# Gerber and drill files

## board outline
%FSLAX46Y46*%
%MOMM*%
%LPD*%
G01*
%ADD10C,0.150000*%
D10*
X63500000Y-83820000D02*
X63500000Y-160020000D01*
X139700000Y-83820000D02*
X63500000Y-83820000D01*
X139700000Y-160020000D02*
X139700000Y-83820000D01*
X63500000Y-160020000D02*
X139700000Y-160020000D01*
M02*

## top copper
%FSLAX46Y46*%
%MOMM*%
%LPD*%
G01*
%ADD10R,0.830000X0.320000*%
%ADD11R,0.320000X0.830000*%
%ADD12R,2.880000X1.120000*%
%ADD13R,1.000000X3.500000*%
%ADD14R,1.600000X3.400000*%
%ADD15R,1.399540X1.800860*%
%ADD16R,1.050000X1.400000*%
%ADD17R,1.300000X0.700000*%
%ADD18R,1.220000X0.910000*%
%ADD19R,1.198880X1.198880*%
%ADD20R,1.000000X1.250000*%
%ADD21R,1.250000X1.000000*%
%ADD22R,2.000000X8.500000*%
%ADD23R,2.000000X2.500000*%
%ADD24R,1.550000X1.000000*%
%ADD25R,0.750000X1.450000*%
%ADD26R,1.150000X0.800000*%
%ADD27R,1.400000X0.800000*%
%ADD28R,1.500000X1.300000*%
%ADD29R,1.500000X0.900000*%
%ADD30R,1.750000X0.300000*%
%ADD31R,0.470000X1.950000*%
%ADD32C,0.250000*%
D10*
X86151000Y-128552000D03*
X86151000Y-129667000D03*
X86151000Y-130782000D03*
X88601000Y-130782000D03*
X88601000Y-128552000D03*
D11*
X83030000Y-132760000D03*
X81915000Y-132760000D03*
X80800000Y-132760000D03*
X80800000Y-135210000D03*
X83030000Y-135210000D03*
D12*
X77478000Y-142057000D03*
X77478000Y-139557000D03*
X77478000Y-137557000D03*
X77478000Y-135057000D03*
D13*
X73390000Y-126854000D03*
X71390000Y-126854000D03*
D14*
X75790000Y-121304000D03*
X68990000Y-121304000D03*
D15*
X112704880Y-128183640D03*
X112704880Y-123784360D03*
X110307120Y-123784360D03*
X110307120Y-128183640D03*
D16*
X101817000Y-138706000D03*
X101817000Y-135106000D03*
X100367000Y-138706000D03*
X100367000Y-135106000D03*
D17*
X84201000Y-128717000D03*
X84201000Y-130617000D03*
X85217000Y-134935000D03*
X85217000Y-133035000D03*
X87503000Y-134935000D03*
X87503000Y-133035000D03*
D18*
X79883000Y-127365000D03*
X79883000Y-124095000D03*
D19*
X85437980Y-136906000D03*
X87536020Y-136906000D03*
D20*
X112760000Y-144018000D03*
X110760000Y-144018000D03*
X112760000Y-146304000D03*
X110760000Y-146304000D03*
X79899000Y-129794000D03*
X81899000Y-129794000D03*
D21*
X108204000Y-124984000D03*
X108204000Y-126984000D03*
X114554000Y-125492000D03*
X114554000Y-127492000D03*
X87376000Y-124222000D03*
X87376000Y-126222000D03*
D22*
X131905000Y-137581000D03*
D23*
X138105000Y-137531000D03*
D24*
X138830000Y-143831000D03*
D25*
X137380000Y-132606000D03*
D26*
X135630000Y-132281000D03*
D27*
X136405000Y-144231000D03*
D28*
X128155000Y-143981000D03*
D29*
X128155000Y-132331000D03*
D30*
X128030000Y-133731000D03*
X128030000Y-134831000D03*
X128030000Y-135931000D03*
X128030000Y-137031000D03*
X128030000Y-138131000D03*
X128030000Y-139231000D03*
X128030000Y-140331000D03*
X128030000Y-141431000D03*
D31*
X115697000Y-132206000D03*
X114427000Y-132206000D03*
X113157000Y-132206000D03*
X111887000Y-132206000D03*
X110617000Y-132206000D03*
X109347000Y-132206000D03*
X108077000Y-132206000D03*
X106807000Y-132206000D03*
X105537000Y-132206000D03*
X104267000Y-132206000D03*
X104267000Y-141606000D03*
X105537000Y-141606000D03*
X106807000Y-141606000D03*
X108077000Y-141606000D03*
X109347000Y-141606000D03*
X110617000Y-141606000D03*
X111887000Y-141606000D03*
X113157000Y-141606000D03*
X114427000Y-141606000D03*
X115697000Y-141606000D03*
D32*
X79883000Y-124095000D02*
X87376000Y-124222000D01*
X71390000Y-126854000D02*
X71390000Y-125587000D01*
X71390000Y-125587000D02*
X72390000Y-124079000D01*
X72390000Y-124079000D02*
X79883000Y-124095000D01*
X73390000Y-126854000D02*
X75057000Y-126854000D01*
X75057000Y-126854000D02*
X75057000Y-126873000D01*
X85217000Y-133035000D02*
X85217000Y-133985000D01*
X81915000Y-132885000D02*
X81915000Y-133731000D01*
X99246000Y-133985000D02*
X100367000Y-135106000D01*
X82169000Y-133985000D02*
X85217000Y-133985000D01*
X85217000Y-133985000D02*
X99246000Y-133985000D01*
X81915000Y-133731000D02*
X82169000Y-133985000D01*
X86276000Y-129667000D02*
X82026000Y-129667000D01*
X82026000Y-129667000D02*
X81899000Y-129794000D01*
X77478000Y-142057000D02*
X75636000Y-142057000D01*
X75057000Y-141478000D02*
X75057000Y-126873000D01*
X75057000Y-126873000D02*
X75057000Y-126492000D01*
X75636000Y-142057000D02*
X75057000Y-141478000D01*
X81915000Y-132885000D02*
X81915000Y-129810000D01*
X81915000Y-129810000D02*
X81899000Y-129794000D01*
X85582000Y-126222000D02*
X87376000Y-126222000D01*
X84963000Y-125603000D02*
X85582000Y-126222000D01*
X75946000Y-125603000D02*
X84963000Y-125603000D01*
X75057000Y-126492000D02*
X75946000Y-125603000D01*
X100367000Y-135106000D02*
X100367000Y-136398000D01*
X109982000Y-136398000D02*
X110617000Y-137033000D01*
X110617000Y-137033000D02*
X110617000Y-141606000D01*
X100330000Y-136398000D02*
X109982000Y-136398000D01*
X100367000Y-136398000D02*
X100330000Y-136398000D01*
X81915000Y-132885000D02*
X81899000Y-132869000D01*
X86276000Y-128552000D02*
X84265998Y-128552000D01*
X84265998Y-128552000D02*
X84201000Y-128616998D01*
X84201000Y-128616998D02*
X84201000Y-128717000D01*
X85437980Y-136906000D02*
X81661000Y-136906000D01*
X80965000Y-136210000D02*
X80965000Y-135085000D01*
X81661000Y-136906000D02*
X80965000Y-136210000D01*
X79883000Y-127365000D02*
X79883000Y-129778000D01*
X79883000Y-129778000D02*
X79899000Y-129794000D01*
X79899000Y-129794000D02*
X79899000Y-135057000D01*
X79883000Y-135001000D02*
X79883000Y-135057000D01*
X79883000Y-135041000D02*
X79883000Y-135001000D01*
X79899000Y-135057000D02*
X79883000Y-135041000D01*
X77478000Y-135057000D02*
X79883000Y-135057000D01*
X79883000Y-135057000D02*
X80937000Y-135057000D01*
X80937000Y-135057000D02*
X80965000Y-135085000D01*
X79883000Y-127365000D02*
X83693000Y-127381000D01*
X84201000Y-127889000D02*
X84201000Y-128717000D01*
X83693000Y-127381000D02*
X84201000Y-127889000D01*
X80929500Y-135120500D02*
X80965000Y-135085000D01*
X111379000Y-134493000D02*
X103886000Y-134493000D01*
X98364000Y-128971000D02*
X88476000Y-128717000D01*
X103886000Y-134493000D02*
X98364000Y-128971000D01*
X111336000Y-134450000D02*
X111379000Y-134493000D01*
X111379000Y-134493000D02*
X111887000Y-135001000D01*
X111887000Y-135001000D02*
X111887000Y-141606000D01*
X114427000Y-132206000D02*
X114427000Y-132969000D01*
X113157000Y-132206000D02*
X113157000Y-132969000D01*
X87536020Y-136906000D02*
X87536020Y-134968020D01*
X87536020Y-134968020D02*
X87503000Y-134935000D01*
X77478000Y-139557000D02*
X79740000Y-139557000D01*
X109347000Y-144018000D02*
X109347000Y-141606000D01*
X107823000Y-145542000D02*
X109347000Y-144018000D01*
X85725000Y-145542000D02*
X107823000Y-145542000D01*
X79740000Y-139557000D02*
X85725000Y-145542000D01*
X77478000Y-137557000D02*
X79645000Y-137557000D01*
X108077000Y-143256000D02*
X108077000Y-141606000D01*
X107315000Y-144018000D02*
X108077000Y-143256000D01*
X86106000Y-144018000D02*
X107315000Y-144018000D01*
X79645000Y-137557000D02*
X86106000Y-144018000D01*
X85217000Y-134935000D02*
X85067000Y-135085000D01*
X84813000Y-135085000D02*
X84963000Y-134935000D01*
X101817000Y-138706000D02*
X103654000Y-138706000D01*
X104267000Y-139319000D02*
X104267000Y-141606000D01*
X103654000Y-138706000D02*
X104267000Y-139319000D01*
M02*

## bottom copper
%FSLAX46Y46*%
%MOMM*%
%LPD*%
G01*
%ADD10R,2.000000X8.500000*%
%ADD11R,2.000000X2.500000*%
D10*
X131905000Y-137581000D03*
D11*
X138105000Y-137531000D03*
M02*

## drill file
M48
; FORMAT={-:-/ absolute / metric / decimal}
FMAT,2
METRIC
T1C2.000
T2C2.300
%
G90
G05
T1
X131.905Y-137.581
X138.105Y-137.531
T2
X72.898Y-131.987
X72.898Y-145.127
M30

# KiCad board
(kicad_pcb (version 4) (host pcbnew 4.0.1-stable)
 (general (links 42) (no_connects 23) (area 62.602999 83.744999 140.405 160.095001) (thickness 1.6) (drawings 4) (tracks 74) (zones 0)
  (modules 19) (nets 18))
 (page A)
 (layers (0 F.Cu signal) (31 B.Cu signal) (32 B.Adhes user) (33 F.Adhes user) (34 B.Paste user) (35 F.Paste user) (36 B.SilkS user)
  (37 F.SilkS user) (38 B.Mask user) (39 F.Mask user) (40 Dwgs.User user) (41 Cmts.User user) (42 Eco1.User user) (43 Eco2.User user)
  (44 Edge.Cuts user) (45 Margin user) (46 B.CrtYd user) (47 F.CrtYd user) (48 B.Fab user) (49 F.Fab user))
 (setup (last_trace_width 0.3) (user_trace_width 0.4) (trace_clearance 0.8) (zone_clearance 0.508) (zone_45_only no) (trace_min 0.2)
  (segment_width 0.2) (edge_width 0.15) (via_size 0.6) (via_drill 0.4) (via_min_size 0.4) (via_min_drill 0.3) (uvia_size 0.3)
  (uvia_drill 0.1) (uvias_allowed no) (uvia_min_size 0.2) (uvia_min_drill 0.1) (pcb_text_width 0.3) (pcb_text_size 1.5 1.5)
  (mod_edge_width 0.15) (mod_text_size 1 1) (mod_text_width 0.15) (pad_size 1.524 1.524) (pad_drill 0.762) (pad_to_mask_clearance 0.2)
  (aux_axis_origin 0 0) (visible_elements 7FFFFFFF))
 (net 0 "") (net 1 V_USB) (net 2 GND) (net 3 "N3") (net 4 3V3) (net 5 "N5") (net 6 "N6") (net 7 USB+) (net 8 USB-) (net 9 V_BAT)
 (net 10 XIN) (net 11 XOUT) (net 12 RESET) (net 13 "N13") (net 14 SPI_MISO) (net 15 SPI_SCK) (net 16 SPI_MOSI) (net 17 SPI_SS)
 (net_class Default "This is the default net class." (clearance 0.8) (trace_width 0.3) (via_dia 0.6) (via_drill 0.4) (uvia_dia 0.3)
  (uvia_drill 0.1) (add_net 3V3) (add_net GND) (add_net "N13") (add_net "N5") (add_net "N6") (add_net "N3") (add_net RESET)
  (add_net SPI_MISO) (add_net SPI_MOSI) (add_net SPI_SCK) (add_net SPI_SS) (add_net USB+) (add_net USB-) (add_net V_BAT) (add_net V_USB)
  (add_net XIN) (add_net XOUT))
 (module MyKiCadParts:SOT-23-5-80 (layer F.Cu) (at 87.376 129.667)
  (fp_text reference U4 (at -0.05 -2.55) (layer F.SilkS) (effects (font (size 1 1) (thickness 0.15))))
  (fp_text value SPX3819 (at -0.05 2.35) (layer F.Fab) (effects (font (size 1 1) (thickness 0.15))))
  (pad 1 smd rect (at -1.225 -1.115) (size 0.83 0.32) (layers F.Cu F.Paste F.Mask) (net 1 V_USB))
  (pad 2 smd rect (at -1.225 0) (size 0.83 0.32) (layers F.Cu F.Paste F.Mask) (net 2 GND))
  (pad 3 smd rect (at -1.225 1.115) (size 0.83 0.32) (layers F.Cu F.Paste F.Mask) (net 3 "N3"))
  (pad 4 smd rect (at 1.225 1.115) (size 0.83 0.32) (layers F.Cu F.Paste F.Mask))
  (pad 5 smd rect (at 1.225 -1.115) (size 0.83 0.32) (layers F.Cu F.Paste F.Mask) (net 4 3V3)))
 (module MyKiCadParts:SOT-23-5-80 (layer F.Cu) (at 81.915 133.985 270)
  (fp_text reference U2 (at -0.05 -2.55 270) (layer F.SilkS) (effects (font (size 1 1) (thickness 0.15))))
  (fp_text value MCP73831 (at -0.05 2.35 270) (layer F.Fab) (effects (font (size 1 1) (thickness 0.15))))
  (pad 1 smd rect (at -1.225 -1.115 270) (size 0.83 0.32) (layers F.Cu F.Paste F.Mask) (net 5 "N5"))
  (pad 2 smd rect (at -1.225 0 270) (size 0.83 0.32) (layers F.Cu F.Paste F.Mask) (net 2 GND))
  (pad 3 smd rect (at -1.225 1.115 270) (size 0.83 0.32) (layers F.Cu F.Paste F.Mask))
  (pad 4 smd rect (at 1.225 1.115 270) (size 0.83 0.32) (layers F.Cu F.Paste F.Mask) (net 1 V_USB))
  (pad 5 smd rect (at 1.225 -1.115 270) (size 0.83 0.32) (layers F.Cu F.Paste F.Mask) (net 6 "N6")))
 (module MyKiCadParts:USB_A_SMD (layer F.Cu) (at 72.898 138.557 270)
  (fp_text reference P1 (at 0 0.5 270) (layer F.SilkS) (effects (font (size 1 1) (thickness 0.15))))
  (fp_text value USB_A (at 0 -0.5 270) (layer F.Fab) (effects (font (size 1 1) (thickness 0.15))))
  (pad "" np_thru_hole circle (at 6.57 0 270) (size 2.3 2.3) (drill 2.3) (layers *.Cu *.Mask F.SilkS))
  (pad 4 smd rect (at 3.5 -4.58 270) (size 1.12 2.88) (layers F.Cu F.Paste F.Mask) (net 2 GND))
  (pad 3 smd rect (at 1 -4.58 270) (size 1.12 2.88) (layers F.Cu F.Paste F.Mask) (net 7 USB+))
  (pad 2 smd rect (at -1 -4.58 270) (size 1.12 2.88) (layers F.Cu F.Paste F.Mask) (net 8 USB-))
  (pad 1 smd rect (at -3.5 -4.58 270) (size 1.12 2.88) (layers F.Cu F.Paste F.Mask) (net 1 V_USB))
  (pad "" np_thru_hole circle (at -6.57 0 270) (size 2.3 2.3) (drill 2.3) (layers *.Cu *.Mask F.SilkS)))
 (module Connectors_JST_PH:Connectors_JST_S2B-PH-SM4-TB (layer F.Cu) (at 72.39 124.079 180)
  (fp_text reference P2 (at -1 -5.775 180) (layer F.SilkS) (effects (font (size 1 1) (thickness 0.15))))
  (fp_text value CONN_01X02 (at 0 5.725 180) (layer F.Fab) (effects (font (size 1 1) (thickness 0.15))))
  (pad 1 smd rect (at -1 -2.775 180) (size 1 3.5) (layers F.Cu F.Paste F.Mask) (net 2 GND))
  (pad 2 smd rect (at 1 -2.775 180) (size 1 3.5) (layers F.Cu F.Paste F.Mask) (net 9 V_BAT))
  (pad "" smd rect (at -3.4 2.775 180) (size 1.6 3.4) (layers F.Cu F.Paste F.Mask))
  (pad "" smd rect (at 3.4 2.775 180) (size 1.6 3.4) (layers F.Cu F.Paste F.Mask)))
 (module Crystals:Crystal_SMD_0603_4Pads (layer F.Cu) (at 111.506 125.984 90)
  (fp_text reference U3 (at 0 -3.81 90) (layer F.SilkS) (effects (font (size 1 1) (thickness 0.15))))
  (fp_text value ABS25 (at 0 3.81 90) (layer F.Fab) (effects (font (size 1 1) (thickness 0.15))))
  (pad 1 smd rect (at -2.19964 1.19888 90) (size 1.80086 1.39954) (layers F.Cu F.Paste F.Mask) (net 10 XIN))
  (pad 2 smd rect (at 2.19964 1.19888 90) (size 1.80086 1.39954) (layers F.Cu F.Paste F.Mask))
  (pad 3 smd rect (at 2.19964 -1.19888 90) (size 1.80086 1.39954) (layers F.Cu F.Paste F.Mask))
  (pad 4 smd rect (at -2.19964 -1.19888 90) (size 1.80086 1.39954) (layers F.Cu F.Paste F.Mask) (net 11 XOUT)))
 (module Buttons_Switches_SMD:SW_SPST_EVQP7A (layer F.Cu) (at 101.092 136.906 270)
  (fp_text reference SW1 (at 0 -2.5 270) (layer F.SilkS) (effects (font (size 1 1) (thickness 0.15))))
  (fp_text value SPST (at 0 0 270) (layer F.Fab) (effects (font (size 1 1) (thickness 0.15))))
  (pad 1 smd rect (at 1.8 -0.725 270) (size 1.4 1.05) (layers F.Cu F.Paste F.Mask) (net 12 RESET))
  (pad 1 smd rect (at -1.8 -0.725 270) (size 1.4 1.05) (layers F.Cu F.Paste F.Mask) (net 12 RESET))
  (pad 2 smd rect (at 1.8 0.725 270) (size 1.4 1.05) (layers F.Cu F.Paste F.Mask) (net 2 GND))
  (pad 2 smd rect (at -1.8 0.725 270) (size 1.4 1.05) (layers F.Cu F.Paste F.Mask) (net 2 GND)))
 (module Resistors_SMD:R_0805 (layer F.Cu) (at 84.201 129.667 270)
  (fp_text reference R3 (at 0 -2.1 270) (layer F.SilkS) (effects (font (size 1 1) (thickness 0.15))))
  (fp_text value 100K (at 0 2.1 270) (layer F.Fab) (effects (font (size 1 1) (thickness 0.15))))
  (pad 1 smd rect (at -0.95 0 270) (size 0.7 1.3) (layers F.Cu F.Paste F.Mask) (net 1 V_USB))
  (pad 2 smd rect (at 0.95 0 270) (size 0.7 1.3) (layers F.Cu F.Paste F.Mask) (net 3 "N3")))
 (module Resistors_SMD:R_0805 (layer F.Cu) (at 85.217 133.985 90)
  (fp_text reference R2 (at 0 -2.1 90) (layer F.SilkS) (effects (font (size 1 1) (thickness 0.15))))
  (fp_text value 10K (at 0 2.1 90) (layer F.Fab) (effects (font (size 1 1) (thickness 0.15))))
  (pad 1 smd rect (at -0.95 0 90) (size 0.7 1.3) (layers F.Cu F.Paste F.Mask) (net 6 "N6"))
  (pad 2 smd rect (at 0.95 0 90) (size 0.7 1.3) (layers F.Cu F.Paste F.Mask) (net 2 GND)))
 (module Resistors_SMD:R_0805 (layer F.Cu) (at 87.503 133.985 90)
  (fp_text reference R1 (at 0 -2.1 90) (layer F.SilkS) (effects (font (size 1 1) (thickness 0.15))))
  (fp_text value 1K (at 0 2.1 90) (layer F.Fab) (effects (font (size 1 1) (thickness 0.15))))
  (pad 1 smd rect (at -0.95 0 90) (size 0.7 1.3) (layers F.Cu F.Paste F.Mask) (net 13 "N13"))
  (pad 2 smd rect (at 0.95 0 90) (size 0.7 1.3) (layers F.Cu F.Paste F.Mask) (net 5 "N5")))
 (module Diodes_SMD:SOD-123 (layer F.Cu) (at 79.883 125.73 90)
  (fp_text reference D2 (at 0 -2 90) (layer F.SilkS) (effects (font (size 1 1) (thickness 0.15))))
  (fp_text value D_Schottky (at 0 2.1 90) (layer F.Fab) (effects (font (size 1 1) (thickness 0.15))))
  (pad 1 smd rect (at -1.635 0 90) (size 0.91 1.22) (layers F.Cu F.Paste F.Mask) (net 1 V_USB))
  (pad 2 smd rect (at 1.635 0 90) (size 0.91 1.22) (layers F.Cu F.Paste F.Mask) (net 9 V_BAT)))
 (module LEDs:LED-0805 (layer F.Cu) (at 86.487 136.906 180)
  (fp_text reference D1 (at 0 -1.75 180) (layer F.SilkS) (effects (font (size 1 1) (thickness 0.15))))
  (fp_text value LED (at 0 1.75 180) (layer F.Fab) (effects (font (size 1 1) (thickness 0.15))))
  (pad 2 smd rect (at 1.04902 0) (size 1.19888 1.19888) (layers F.Cu F.Paste F.Mask) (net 1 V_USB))
  (pad 1 smd rect (at -1.04902 0) (size 1.19888 1.19888) (layers F.Cu F.Paste F.Mask) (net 13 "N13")))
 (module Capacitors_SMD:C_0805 (layer F.Cu) (at 111.76 144.018 180)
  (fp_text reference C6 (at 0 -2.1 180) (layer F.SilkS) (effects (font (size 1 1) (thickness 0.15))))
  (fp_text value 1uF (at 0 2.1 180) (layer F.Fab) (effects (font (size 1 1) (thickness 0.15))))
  (pad 1 smd rect (at -1 0 180) (size 1 1.25) (layers F.Cu F.Paste F.Mask) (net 4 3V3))
  (pad 2 smd rect (at 1 0 180) (size 1 1.25) (layers F.Cu F.Paste F.Mask) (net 2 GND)))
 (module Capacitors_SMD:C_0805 (layer F.Cu) (at 111.76 146.304 180)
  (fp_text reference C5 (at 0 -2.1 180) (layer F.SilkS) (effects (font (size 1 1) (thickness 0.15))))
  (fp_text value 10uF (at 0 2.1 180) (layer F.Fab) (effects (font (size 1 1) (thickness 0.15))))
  (pad 1 smd rect (at -1 0 180) (size 1 1.25) (layers F.Cu F.Paste F.Mask) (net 4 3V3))
  (pad 2 smd rect (at 1 0 180) (size 1 1.25) (layers F.Cu F.Paste F.Mask) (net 2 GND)))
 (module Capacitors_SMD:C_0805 (layer F.Cu) (at 80.899 129.794)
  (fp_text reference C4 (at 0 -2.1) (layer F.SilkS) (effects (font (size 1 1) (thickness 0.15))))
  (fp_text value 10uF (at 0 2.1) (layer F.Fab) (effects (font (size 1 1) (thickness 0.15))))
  (pad 1 smd rect (at -1 0) (size 1 1.25) (layers F.Cu F.Paste F.Mask) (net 1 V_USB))
  (pad 2 smd rect (at 1 0) (size 1 1.25) (layers F.Cu F.Paste F.Mask) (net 2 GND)))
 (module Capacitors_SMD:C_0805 (layer F.Cu) (at 108.204 125.984 270)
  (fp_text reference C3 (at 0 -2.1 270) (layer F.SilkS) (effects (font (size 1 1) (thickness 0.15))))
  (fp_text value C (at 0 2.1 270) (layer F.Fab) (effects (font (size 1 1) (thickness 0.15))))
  (pad 1 smd rect (at -1 0 270) (size 1 1.25) (layers F.Cu F.Paste F.Mask) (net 2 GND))
  (pad 2 smd rect (at 1 0 270) (size 1 1.25) (layers F.Cu F.Paste F.Mask) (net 11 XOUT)))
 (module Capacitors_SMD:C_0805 (layer F.Cu) (at 114.554 126.492 270)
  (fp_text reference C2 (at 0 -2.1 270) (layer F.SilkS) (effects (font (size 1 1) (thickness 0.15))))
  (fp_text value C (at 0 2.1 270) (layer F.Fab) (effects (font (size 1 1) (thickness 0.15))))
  (pad 1 smd rect (at -1 0 270) (size 1 1.25) (layers F.Cu F.Paste F.Mask) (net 2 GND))
  (pad 2 smd rect (at 1 0 270) (size 1 1.25) (layers F.Cu F.Paste F.Mask) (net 10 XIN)))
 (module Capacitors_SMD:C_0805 (layer F.Cu) (at 87.376 125.222 270)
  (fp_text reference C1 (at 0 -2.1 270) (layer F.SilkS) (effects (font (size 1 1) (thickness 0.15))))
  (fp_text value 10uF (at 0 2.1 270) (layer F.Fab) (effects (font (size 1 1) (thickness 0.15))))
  (pad 1 smd rect (at -1 0 270) (size 1 1.25) (layers F.Cu F.Paste F.Mask) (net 9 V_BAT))
  (pad 2 smd rect (at 1 0 270) (size 1 1.25) (layers F.Cu F.Paste F.Mask) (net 2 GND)))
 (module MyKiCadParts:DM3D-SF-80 (layer F.Cu) (at 128.905 133.731 270)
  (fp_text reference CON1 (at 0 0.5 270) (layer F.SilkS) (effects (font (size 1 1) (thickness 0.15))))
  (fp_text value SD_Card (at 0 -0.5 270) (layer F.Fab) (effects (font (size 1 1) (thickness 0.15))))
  (pad "" np_thru_hole rect (at 3.85 -3 270) (size 8.5 2) (drill 2) (layers *.Cu *.Mask F.SilkS))
  (pad "" np_thru_hole rect (at 3.8 -9.2 270) (size 2.5 2) (drill 2) (layers *.Cu *.Mask F.SilkS))
  (pad "" smd rect (at 10.1 -9.925 270) (size 1 1.55) (layers F.Cu F.Paste F.Mask))
  (pad "" smd rect (at -1.125 -8.475 270) (size 1.45 0.75) (layers F.Cu F.Paste F.Mask))
  (pad "" smd rect (at -1.45 -6.725 270) (size 0.8 1.15) (layers F.Cu F.Paste F.Mask))
  (pad "" smd rect (at 10.5 -7.5 270) (size 0.8 1.4) (layers F.Cu F.Paste F.Mask))
  (pad "" smd rect (at 10.25 0.75 270) (size 1.3 1.5) (layers F.Cu F.Paste F.Mask))
  (pad "" smd rect (at -1.4 0.75 270) (size 0.9 1.5) (layers F.Cu F.Paste F.Mask))
  (pad 8 smd rect (at 0 0.875 270) (size 0.3 1.75) (layers F.Cu F.Paste F.Mask))
  (pad 7 smd rect (at 1.1 0.875 270) (size 0.3 1.75) (layers F.Cu F.Paste F.Mask) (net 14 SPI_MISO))
  (pad 6 smd rect (at 2.2 0.875 270) (size 0.3 1.75) (layers F.Cu F.Paste F.Mask) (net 2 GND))
  (pad 5 smd rect (at 3.3 0.875 270) (size 0.3 1.75) (layers F.Cu F.Paste F.Mask) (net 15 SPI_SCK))
  (pad 4 smd rect (at 4.4 0.875 270) (size 0.3 1.75) (layers F.Cu F.Paste F.Mask) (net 4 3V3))
  (pad 3 smd rect (at 5.5 0.875 270) (size 0.3 1.75) (layers F.Cu F.Paste F.Mask) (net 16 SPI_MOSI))
  (pad 2 smd rect (at 6.6 0.875 270) (size 0.3 1.75) (layers F.Cu F.Paste F.Mask) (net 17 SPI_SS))
  (pad 1 smd rect (at 7.7 0.875 270) (size 0.3 1.75) (layers F.Cu F.Paste F.Mask)))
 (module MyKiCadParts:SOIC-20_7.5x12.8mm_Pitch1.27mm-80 (layer F.Cu) (at 109.982 136.906 270)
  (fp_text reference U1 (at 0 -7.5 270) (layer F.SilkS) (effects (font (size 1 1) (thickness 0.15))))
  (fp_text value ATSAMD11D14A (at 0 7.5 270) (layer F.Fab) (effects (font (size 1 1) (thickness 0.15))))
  (pad 1 smd rect (at -4.7 -5.715 270) (size 1.95 0.47) (layers F.Cu F.Paste F.Mask) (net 17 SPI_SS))
  (pad 2 smd rect (at -4.7 -4.445 270) (size 1.95 0.47) (layers F.Cu F.Paste F.Mask) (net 16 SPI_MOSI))
  (pad 3 smd rect (at -4.7 -3.175 270) (size 1.95 0.47) (layers F.Cu F.Paste F.Mask) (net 15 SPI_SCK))
  (pad 4 smd rect (at -4.7 -1.905 270) (size 1.95 0.47) (layers F.Cu F.Paste F.Mask) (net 10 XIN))
  (pad 5 smd rect (at -4.7 -0.635 270) (size 1.95 0.47) (layers F.Cu F.Paste F.Mask) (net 11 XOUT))
  (pad 6 smd rect (at -4.7 0.635 270) (size 1.95 0.47) (layers F.Cu F.Paste F.Mask))
  (pad 7 smd rect (at -4.7 1.905 270) (size 1.95 0.47) (layers F.Cu F.Paste F.Mask))
  (pad 8 smd rect (at -4.7 3.175 270) (size 1.95 0.47) (layers F.Cu F.Paste F.Mask))
  (pad 9 smd rect (at -4.7 4.445 270) (size 1.95 0.47) (layers F.Cu F.Paste F.Mask))
  (pad 10 smd rect (at -4.7 5.715 270) (size 1.95 0.47) (layers F.Cu F.Paste F.Mask))
  (pad 11 smd rect (at 4.7 5.715 270) (size 1.95 0.47) (layers F.Cu F.Paste F.Mask) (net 12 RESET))
  (pad 12 smd rect (at 4.7 4.445 270) (size 1.95 0.47) (layers F.Cu F.Paste F.Mask))
  (pad 13 smd rect (at 4.7 3.175 270) (size 1.95 0.47) (layers F.Cu F.Paste F.Mask))
  (pad 14 smd rect (at 4.7 1.905 270) (size 1.95 0.47) (layers F.Cu F.Paste F.Mask) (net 8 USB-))
  (pad 15 smd rect (at 4.7 0.635 270) (size 1.95 0.47) (layers F.Cu F.Paste F.Mask) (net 7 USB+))
  (pad 16 smd rect (at 4.7 -0.635 270) (size 1.95 0.47) (layers F.Cu F.Paste F.Mask) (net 2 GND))
  (pad 17 smd rect (at 4.7 -1.905 270) (size 1.95 0.47) (layers F.Cu F.Paste F.Mask) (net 4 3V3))
  (pad 18 smd rect (at 4.7 -3.175 270) (size 1.95 0.47) (layers F.Cu F.Paste F.Mask))
  (pad 19 smd rect (at 4.7 -4.445 270) (size 1.95 0.47) (layers F.Cu F.Paste F.Mask))
  (pad 20 smd rect (at 4.7 -5.715 270) (size 1.95 0.47) (layers F.Cu F.Paste F.Mask) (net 14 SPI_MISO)))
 (gr_line (start 63.5 83.82) (end 63.5 160.02) (angle 90) (layer Edge.Cuts) (width 0.15))
 (gr_line (start 139.7 83.82) (end 63.5 83.82) (angle 90) (layer Edge.Cuts) (width 0.15))
 (gr_line (start 139.7 160.02) (end 139.7 83.82) (angle 90) (layer Edge.Cuts) (width 0.15))
 (gr_line (start 63.5 160.02) (end 139.7 160.02) (angle 90) (layer Edge.Cuts) (width 0.15))
 (segment (start 79.883 124.095) (end 87.376 124.222) (width 0.25) (layer F.Cu) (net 9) (status 10))
 (segment (start 71.39 126.854) (end 71.39 125.587) (width 0.25) (layer F.Cu) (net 9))
 (segment (start 71.39 125.587) (end 72.39 124.079) (width 0.25) (layer F.Cu) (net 9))
 (segment (start 72.39 124.079) (end 79.883 124.095) (width 0.25) (layer F.Cu) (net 9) (status 20))
 (segment (start 73.39 126.854) (end 75.057 126.854) (width 0.25) (layer F.Cu) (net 2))
 (segment (start 75.057 126.854) (end 75.057 126.873) (width 0.25) (layer F.Cu) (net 2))
 (segment (start 85.217 133.035) (end 85.217 133.985) (width 0.25) (layer F.Cu) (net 2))
 (segment (start 81.915 132.885) (end 81.915 133.731) (width 0.25) (layer F.Cu) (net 2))
 (segment (start 99.246 133.985) (end 100.367 135.106) (width 0.25) (layer F.Cu) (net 2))
 (segment (start 82.169 133.985) (end 85.217 133.985) (width 0.25) (layer F.Cu) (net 2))
 (segment (start 85.217 133.985) (end 99.246 133.985) (width 0.25) (layer F.Cu) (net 2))
 (segment (start 81.915 133.731) (end 82.169 133.985) (width 0.25) (layer F.Cu) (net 2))
 (segment (start 86.276 129.667) (end 82.026 129.667) (width 0.25) (layer F.Cu) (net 2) (status 20))
 (segment (start 82.026 129.667) (end 81.899 129.794) (width 0.25) (layer F.Cu) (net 2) (status 30))
 (segment (start 77.478 142.057) (end 75.636 142.057) (width 0.25) (layer F.Cu) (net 2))
 (segment (start 75.057 141.478) (end 75.057 126.873) (width 0.25) (layer F.Cu) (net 2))
 (segment (start 75.057 126.873) (end 75.057 126.492) (width 0.25) (layer F.Cu) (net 2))
 (segment (start 75.636 142.057) (end 75.057 141.478) (width 0.25) (layer F.Cu) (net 2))
 (segment (start 81.915 132.885) (end 81.915 129.81) (width 0.25) (layer F.Cu) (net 2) (status 20))
 (segment (start 81.915 129.81) (end 81.899 129.794) (width 0.25) (layer F.Cu) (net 2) (status 30))
 (segment (start 85.582 126.222) (end 87.376 126.222) (width 0.25) (layer F.Cu) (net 2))
 (segment (start 84.963 125.603) (end 85.582 126.222) (width 0.25) (layer F.Cu) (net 2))
 (segment (start 75.946 125.603) (end 84.963 125.603) (width 0.25) (layer F.Cu) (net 2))
 (segment (start 75.057 126.492) (end 75.946 125.603) (width 0.25) (layer F.Cu) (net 2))
 (segment (start 100.367 135.106) (end 100.367 136.398) (width 0.25) (layer F.Cu) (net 2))
 (segment (start 109.982 136.398) (end 110.617 137.033) (width 0.25) (layer F.Cu) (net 2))
 (segment (start 110.617 137.033) (end 110.617 141.606) (width 0.25) (layer F.Cu) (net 2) (status 20))
 (segment (start 100.33 136.398) (end 109.982 136.398) (width 0.25) (layer F.Cu) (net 2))
 (segment (start 100.367 136.398) (end 100.33 136.398) (width 0.25) (layer F.Cu) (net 2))
 (segment (start 81.915 132.885) (end 81.899 132.869) (width 0.25) (layer F.Cu) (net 2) (status 30))
 (segment (start 86.276 128.552) (end 84.265998 128.552) (width 0.25) (layer F.Cu) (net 1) (status 10))
 (segment (start 84.265998 128.552) (end 84.201 128.616998) (width 0.25) (layer F.Cu) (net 1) (status 30))
 (segment (start 84.201 128.616998) (end 84.201 128.717) (width 0.25) (layer F.Cu) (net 1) (status 30))
 (segment (start 85.43798 136.906) (end 81.661 136.906) (width 0.25) (layer F.Cu) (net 1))
 (segment (start 80.965 136.21) (end 80.965 135.085) (width 0.25) (layer F.Cu) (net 1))
 (segment (start 81.661 136.906) (end 80.965 136.21) (width 0.25) (layer F.Cu) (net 1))
 (segment (start 79.883 127.365) (end 79.883 129.778) (width 0.25) (layer F.Cu) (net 1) (status 10))
 (segment (start 79.883 129.778) (end 79.899 129.794) (width 0.25) (layer F.Cu) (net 1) (status 30))
 (segment (start 79.899 129.794) (end 79.899 135.057) (width 0.25) (layer F.Cu) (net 1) (status 10))
 (segment (start 79.883 135.001) (end 79.883 135.057) (width 0.25) (layer F.Cu) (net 1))
 (segment (start 79.883 135.041) (end 79.883 135.001) (width 0.25) (layer F.Cu) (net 1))
 (segment (start 79.899 135.057) (end 79.883 135.041) (width 0.25) (layer F.Cu) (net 1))
 (segment (start 77.478 135.057) (end 79.883 135.057) (width 0.25) (layer F.Cu) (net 1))
 (segment (start 79.883 135.057) (end 80.937 135.057) (width 0.25) (layer F.Cu) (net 1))
 (segment (start 80.937 135.057) (end 80.965 135.085) (width 0.25) (layer F.Cu) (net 1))
 (segment (start 79.883 127.365) (end 83.693 127.381) (width 0.25) (layer F.Cu) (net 1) (status 10))
 (segment (start 84.201 127.889) (end 84.201 128.717) (width 0.25) (layer F.Cu) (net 1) (status 20))
 (segment (start 83.693 127.381) (end 84.201 127.889) (width 0.25) (layer F.Cu) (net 1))
 (segment (start 80.9295 135.1205) (end 80.965 135.085) (width 0.25) (layer F.Cu) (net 1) (status 30))
 (segment (start 111.379 134.493) (end 103.886 134.493) (width 0.25) (layer F.Cu) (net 4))
 (segment (start 98.364 128.971) (end 88.476 128.717) (width 0.25) (layer F.Cu) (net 4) (status 20))
 (segment (start 103.886 134.493) (end 98.364 128.971) (width 0.25) (layer F.Cu) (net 4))
 (segment (start 111.336 134.45) (end 111.379 134.493) (width 0.25) (layer F.Cu) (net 4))
 (segment (start 111.379 134.493) (end 111.887 135.001) (width 0.25) (layer F.Cu) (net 4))
 (segment (start 111.887 135.001) (end 111.887 141.606) (width 0.25) (layer F.Cu) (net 4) (status 20))
 (segment (start 114.427 132.206) (end 114.427 132.969) (width 0.25) (layer F.Cu) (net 16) (status 30))
 (segment (start 113.157 132.206) (end 113.157 132.969) (width 0.25) (layer F.Cu) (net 15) (status 30))
 (segment (start 87.53602 136.906) (end 87.53602 134.96802) (width 0.25) (layer F.Cu) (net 13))
 (segment (start 87.53602 134.96802) (end 87.503 134.935) (width 0.25) (layer F.Cu) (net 13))
 (segment (start 77.478 139.557) (end 79.74 139.557) (width 0.25) (layer F.Cu) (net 7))
 (segment (start 109.347 144.018) (end 109.347 141.606) (width 0.25) (layer F.Cu) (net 7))
 (segment (start 107.823 145.542) (end 109.347 144.018) (width 0.25) (layer F.Cu) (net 7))
 (segment (start 85.725 145.542) (end 107.823 145.542) (width 0.25) (layer F.Cu) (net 7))
 (segment (start 79.74 139.557) (end 85.725 145.542) (width 0.25) (layer F.Cu) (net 7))
 (segment (start 77.478 137.557) (end 79.645 137.557) (width 0.25) (layer F.Cu) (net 8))
 (segment (start 108.077 143.256) (end 108.077 141.606) (width 0.25) (layer F.Cu) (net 8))
 (segment (start 107.315 144.018) (end 108.077 143.256) (width 0.25) (layer F.Cu) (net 8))
 (segment (start 86.106 144.018) (end 107.315 144.018) (width 0.25) (layer F.Cu) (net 8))
 (segment (start 79.645 137.557) (end 86.106 144.018) (width 0.25) (layer F.Cu) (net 8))
 (segment (start 85.217 134.935) (end 85.067 135.085) (width 0.25) (layer F.Cu) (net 6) (status 30))
 (segment (start 84.813 135.085) (end 84.963 134.935) (width 0.25) (layer F.Cu) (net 6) (status 30))
 (segment (start 101.817 138.706) (end 103.654 138.706) (width 0.25) (layer F.Cu) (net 12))
 (segment (start 104.267 139.319) (end 104.267 141.606) (width 0.25) (layer F.Cu) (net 12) (status 20))
 (segment (start 103.654 138.706) (end 104.267 139.319) (width 0.25) (layer F.Cu) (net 12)))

